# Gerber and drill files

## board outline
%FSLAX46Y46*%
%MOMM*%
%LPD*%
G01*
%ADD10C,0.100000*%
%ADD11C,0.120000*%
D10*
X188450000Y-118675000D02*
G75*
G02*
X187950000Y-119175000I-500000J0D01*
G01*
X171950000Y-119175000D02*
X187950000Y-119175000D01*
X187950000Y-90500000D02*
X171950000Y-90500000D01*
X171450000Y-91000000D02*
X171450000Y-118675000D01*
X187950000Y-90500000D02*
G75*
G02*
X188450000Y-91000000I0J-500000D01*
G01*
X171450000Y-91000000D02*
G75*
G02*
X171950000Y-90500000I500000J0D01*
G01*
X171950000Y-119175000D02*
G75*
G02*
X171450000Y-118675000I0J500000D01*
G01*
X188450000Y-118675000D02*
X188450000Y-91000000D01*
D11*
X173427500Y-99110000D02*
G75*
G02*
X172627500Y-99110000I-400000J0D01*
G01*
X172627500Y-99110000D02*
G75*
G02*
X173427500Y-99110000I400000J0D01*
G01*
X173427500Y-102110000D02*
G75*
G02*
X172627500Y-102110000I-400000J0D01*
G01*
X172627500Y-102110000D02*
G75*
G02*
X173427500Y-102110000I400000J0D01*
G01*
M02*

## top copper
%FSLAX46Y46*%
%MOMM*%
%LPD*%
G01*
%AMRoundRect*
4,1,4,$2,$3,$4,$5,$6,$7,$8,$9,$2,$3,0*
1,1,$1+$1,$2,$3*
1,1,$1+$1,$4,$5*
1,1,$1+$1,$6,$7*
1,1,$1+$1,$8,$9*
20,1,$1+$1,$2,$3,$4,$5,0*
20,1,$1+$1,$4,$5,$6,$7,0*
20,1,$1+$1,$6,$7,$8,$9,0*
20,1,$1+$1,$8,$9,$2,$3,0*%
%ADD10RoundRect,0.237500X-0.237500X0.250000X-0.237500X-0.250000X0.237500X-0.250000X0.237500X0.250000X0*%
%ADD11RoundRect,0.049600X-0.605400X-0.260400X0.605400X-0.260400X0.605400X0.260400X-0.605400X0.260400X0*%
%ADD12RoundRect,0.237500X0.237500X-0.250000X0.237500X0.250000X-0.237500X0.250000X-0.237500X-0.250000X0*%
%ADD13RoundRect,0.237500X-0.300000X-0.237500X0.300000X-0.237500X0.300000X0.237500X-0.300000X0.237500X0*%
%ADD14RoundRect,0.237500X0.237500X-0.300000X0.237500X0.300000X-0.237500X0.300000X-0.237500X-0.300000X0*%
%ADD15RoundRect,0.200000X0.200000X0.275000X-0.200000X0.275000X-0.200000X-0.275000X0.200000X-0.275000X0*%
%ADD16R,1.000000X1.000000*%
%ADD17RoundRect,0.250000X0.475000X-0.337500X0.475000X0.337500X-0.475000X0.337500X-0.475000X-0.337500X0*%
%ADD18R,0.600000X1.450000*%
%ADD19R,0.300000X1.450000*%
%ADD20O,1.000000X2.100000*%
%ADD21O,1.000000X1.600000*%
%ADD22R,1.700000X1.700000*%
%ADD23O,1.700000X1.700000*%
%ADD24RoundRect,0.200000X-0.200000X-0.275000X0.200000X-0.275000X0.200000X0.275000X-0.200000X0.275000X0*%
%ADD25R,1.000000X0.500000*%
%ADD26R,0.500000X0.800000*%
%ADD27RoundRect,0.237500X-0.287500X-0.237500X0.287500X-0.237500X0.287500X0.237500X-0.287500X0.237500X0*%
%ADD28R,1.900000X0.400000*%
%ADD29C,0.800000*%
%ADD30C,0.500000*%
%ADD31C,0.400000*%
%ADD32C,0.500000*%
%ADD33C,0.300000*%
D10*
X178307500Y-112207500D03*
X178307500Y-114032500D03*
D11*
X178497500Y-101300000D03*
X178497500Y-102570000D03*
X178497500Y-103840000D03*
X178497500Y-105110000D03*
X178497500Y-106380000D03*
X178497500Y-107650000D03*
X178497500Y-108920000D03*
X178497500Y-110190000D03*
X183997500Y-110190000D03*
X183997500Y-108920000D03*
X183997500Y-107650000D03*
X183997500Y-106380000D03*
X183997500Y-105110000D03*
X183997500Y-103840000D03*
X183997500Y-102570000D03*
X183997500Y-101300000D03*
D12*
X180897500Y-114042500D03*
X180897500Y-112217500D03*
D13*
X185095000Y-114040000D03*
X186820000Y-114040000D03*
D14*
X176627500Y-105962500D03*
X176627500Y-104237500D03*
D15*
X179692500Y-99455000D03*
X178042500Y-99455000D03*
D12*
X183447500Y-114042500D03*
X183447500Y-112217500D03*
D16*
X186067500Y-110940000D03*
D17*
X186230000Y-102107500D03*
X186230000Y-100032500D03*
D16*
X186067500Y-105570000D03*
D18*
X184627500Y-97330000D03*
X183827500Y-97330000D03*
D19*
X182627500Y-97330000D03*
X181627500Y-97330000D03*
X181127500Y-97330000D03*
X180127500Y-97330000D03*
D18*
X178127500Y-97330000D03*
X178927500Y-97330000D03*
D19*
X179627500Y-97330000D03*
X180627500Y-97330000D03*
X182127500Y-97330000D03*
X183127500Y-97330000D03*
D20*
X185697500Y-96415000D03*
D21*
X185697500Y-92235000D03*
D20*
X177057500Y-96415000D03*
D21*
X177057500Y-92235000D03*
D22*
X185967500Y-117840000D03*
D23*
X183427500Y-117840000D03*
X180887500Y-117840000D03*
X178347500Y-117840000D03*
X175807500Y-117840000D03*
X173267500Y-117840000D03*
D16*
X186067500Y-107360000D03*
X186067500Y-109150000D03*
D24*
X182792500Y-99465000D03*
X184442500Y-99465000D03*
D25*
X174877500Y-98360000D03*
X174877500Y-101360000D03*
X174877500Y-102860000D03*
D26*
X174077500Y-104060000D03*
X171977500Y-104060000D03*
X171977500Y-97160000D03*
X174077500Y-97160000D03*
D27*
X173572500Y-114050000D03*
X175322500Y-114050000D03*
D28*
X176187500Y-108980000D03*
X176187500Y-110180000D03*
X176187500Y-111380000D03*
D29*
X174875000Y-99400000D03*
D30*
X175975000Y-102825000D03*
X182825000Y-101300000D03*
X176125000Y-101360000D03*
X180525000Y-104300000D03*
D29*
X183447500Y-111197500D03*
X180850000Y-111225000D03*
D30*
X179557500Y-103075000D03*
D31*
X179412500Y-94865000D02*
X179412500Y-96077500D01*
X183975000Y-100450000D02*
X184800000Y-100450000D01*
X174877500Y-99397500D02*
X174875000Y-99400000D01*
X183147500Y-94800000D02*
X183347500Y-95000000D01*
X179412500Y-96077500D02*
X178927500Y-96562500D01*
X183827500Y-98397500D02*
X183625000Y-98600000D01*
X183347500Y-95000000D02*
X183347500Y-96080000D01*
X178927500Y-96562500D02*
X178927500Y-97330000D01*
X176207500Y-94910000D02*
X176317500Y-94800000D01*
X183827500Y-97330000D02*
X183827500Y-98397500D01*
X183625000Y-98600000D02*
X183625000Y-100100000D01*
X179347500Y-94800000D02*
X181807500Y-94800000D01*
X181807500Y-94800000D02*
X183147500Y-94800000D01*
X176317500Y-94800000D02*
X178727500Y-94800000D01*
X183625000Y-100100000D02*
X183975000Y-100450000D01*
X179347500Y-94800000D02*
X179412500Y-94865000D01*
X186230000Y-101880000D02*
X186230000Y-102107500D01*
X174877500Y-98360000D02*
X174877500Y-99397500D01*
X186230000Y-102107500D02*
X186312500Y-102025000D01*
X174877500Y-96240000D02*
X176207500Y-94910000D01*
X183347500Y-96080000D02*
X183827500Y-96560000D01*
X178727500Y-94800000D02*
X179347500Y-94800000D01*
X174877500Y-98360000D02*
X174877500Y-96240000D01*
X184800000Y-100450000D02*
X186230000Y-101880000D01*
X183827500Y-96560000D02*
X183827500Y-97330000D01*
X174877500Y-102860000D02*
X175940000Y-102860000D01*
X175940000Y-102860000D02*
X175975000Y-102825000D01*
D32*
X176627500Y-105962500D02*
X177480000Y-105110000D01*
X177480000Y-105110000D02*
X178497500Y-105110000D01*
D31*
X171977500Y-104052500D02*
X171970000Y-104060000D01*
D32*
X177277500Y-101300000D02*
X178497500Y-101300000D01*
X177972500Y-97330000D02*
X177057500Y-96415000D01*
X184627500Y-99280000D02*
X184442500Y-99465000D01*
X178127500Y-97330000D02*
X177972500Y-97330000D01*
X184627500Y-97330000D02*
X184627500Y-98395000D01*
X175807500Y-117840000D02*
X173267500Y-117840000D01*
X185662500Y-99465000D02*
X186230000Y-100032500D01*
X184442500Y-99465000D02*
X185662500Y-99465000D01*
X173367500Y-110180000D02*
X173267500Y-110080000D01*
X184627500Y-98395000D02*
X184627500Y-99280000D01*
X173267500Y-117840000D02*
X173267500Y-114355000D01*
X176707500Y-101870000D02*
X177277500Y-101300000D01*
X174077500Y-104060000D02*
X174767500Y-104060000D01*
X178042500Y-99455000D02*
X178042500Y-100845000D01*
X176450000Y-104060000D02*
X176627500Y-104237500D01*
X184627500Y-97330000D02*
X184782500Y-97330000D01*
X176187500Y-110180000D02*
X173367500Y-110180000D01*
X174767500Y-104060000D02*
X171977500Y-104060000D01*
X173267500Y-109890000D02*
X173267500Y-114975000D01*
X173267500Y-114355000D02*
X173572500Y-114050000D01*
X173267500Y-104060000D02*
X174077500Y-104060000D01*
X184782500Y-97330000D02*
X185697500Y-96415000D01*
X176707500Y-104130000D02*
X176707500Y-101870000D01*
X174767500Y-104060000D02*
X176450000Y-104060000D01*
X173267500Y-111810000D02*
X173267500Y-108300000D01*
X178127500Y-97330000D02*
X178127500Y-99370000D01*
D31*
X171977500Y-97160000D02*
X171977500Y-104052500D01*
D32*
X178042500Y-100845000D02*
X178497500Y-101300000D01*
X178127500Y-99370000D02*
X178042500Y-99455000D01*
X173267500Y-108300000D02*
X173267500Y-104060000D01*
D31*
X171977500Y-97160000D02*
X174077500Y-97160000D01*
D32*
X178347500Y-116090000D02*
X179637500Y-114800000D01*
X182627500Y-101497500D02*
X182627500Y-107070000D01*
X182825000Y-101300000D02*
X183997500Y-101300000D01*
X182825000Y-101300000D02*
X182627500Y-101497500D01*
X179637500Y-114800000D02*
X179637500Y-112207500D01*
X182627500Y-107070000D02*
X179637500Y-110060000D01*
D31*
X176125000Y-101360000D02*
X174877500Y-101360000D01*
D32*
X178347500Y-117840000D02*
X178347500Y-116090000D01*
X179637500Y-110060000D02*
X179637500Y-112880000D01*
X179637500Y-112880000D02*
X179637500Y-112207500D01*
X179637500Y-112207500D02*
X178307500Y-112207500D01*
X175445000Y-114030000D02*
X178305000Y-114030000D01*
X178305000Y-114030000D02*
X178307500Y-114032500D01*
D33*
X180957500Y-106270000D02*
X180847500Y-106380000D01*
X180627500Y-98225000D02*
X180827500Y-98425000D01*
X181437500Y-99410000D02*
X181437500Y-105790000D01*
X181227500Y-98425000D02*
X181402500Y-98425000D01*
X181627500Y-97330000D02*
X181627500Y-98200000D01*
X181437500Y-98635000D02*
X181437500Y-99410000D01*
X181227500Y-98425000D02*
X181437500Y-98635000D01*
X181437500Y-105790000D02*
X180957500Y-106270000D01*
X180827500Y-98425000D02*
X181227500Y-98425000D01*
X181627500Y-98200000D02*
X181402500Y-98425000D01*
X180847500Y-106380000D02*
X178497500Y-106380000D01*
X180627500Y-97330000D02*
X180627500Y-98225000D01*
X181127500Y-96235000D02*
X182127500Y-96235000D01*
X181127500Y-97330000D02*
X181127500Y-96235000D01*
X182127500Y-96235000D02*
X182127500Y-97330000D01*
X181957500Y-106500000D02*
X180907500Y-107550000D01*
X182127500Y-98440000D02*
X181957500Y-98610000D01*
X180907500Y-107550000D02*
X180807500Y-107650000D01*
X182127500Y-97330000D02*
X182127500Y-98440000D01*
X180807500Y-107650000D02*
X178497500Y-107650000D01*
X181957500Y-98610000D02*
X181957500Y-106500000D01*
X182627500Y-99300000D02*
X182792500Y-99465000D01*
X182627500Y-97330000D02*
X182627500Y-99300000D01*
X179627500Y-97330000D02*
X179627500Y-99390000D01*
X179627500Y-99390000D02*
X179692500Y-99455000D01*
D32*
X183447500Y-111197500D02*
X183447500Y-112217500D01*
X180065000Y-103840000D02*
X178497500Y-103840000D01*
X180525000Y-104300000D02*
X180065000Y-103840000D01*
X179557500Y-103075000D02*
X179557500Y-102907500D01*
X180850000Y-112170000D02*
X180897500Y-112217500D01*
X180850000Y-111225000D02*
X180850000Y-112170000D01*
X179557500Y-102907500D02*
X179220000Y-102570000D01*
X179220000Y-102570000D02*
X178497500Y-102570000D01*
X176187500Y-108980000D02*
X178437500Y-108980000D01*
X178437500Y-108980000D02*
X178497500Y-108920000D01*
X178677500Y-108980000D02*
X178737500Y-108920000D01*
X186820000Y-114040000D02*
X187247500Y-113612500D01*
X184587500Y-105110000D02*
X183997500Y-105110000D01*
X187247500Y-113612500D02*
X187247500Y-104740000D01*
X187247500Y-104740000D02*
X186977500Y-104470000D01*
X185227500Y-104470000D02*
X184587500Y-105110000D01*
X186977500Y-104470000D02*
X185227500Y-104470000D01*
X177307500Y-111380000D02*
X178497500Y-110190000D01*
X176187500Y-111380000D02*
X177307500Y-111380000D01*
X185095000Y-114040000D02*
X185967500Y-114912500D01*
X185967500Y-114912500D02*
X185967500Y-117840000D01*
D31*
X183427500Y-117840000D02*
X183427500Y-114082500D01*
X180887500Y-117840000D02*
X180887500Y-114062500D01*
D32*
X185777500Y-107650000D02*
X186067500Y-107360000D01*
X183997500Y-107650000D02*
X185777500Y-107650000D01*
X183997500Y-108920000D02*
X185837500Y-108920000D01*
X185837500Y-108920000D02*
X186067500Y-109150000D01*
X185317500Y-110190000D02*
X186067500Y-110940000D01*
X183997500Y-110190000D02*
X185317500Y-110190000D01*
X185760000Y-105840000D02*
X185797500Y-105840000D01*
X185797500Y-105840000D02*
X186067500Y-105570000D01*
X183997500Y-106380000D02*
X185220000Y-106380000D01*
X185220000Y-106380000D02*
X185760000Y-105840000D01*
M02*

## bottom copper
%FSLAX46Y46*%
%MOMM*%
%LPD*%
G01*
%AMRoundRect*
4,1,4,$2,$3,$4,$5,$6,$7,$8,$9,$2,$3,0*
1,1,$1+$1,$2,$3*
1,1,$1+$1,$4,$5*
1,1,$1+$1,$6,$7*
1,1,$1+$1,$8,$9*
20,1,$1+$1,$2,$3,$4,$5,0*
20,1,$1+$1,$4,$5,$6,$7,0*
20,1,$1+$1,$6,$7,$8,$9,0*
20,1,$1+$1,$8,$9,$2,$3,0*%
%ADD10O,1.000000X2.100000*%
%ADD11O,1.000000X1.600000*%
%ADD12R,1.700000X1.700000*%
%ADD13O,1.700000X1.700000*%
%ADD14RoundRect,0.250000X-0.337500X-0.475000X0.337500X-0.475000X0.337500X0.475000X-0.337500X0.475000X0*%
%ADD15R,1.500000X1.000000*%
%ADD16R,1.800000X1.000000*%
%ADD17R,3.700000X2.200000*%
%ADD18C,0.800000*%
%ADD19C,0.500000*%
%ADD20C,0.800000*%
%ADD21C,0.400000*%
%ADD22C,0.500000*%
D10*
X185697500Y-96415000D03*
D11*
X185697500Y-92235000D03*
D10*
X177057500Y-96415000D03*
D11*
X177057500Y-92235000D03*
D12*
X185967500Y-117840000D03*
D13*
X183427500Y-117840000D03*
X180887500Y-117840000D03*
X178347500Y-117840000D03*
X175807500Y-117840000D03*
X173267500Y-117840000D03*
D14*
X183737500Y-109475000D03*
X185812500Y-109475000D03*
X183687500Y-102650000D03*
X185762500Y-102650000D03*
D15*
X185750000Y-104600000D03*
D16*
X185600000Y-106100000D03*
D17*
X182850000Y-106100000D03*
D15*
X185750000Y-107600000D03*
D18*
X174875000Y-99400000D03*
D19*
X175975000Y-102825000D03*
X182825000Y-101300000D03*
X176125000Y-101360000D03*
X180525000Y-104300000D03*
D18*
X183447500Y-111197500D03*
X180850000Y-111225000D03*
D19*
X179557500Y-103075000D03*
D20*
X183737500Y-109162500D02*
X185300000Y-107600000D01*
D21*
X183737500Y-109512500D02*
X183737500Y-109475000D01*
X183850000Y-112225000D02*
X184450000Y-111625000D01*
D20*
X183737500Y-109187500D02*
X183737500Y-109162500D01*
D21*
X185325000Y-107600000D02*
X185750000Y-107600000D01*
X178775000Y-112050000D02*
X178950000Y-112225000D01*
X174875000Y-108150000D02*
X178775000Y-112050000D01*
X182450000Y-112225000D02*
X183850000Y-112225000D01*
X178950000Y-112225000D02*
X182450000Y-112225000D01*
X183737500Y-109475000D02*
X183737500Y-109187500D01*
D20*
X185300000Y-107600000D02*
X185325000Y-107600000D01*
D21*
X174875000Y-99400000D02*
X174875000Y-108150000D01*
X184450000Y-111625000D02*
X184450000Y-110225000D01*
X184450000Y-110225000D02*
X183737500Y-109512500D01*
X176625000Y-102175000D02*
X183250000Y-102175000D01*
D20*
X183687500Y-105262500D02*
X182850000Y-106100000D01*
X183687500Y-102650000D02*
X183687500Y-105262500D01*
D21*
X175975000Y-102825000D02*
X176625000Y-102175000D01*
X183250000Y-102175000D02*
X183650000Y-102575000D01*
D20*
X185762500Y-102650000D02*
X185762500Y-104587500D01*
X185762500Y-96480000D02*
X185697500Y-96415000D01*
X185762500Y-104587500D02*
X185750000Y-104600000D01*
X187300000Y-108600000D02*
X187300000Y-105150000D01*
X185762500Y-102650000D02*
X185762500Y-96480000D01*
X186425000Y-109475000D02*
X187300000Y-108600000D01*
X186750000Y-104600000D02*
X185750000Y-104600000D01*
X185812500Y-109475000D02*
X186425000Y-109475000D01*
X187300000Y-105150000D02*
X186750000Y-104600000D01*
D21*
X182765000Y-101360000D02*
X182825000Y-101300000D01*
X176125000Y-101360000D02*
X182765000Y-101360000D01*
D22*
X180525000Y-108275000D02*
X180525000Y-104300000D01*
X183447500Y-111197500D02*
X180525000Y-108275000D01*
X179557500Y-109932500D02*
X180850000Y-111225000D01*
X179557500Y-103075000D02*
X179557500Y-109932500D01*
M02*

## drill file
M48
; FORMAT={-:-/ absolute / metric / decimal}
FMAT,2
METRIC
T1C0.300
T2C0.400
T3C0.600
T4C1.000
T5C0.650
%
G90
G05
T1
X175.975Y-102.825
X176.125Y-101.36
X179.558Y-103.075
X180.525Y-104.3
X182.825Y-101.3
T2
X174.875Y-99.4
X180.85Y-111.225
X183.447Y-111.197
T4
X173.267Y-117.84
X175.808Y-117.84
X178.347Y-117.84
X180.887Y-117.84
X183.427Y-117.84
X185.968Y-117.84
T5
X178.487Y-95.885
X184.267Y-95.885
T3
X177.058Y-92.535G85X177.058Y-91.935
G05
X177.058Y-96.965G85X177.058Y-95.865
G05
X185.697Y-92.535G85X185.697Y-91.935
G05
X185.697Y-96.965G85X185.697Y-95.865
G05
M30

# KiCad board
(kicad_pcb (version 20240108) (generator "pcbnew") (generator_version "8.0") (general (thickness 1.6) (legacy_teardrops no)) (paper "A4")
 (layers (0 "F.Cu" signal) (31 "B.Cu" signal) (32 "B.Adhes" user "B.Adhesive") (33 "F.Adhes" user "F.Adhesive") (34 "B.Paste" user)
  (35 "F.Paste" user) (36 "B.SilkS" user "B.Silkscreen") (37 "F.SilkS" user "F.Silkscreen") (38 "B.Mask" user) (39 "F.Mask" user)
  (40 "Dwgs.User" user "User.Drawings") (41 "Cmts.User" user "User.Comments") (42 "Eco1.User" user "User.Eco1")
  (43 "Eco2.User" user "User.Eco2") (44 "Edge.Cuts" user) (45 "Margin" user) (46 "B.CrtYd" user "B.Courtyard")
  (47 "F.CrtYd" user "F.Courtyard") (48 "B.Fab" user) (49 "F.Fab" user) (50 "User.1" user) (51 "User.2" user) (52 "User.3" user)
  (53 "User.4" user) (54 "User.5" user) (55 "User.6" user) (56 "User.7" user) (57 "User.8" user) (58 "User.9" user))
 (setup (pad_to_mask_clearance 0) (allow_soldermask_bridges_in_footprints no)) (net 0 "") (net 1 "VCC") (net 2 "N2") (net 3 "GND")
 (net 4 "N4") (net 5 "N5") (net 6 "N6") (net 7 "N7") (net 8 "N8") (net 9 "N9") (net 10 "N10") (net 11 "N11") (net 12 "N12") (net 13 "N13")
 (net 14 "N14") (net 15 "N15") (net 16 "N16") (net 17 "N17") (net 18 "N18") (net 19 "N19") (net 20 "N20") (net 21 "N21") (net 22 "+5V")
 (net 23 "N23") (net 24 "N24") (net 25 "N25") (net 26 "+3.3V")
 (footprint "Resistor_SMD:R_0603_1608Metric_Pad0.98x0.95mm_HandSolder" (layer "F.Cu") (at 178.3075 113.12 -90)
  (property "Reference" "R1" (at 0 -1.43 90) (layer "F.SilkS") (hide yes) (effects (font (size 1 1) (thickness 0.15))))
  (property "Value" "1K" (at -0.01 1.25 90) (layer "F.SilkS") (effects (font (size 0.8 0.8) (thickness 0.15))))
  (pad "1" smd roundrect (at -0.9125 0 270) (size 0.975 0.95) (layers "F.Cu" "F.Paste" "F.Mask") (roundrect_rratio 0.25) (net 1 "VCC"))
  (pad "2" smd roundrect (at 0.9125 0 270) (size 0.975 0.95) (layers "F.Cu" "F.Paste" "F.Mask") (roundrect_rratio 0.25) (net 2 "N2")))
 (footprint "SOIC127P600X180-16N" (layer "F.Cu") (at 181.2475 105.745)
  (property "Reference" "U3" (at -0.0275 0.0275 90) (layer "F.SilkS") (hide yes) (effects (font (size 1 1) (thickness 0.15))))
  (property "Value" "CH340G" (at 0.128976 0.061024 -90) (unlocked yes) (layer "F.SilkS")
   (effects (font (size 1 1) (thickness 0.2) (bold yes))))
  (pad "1" smd roundrect (at -2.75 -4.445) (size 1.31 0.62) (layers "F.Cu" "F.Paste" "F.Mask") (roundrect_rratio 0.08) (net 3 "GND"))
  (pad "2" smd roundrect (at -2.75 -3.175) (size 1.31 0.62) (layers "F.Cu" "F.Paste" "F.Mask") (roundrect_rratio 0.08) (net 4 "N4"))
  (pad "3" smd roundrect (at -2.75 -1.905) (size 1.31 0.62) (layers "F.Cu" "F.Paste" "F.Mask") (roundrect_rratio 0.08) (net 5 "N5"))
  (pad "4" smd roundrect (at -2.75 -0.635) (size 1.31 0.62) (layers "F.Cu" "F.Paste" "F.Mask") (roundrect_rratio 0.08) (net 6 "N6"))
  (pad "5" smd roundrect (at -2.75 0.635) (size 1.31 0.62) (layers "F.Cu" "F.Paste" "F.Mask") (roundrect_rratio 0.08) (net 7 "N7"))
  (pad "6" smd roundrect (at -2.75 1.905) (size 1.31 0.62) (layers "F.Cu" "F.Paste" "F.Mask") (roundrect_rratio 0.08) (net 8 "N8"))
  (pad "7" smd roundrect (at -2.75 3.175) (size 1.31 0.62) (layers "F.Cu" "F.Paste" "F.Mask") (roundrect_rratio 0.08) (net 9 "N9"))
  (pad "8" smd roundrect (at -2.75 4.445) (size 1.31 0.62) (layers "F.Cu" "F.Paste" "F.Mask") (roundrect_rratio 0.08) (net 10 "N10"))
  (pad "9" smd roundrect (at 2.75 4.445) (size 1.31 0.62) (layers "F.Cu" "F.Paste" "F.Mask") (roundrect_rratio 0.08) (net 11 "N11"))
  (pad "10" smd roundrect (at 2.75 3.175) (size 1.31 0.62) (layers "F.Cu" "F.Paste" "F.Mask") (roundrect_rratio 0.08) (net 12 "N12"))
  (pad "11" smd roundrect (at 2.75 1.905) (size 1.31 0.62) (layers "F.Cu" "F.Paste" "F.Mask") (roundrect_rratio 0.08) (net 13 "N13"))
  (pad "12" smd roundrect (at 2.75 0.635) (size 1.31 0.62) (layers "F.Cu" "F.Paste" "F.Mask") (roundrect_rratio 0.08) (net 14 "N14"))
  (pad "13" smd roundrect (at 2.75 -0.635) (size 1.31 0.62) (layers "F.Cu" "F.Paste" "F.Mask") (roundrect_rratio 0.08) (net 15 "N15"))
  (pad "14" smd roundrect (at 2.75 -1.905) (size 1.31 0.62) (layers "F.Cu" "F.Paste" "F.Mask") (roundrect_rratio 0.08) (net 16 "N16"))
  (pad "15" smd roundrect (at 2.75 -3.175) (size 1.31 0.62) (layers "F.Cu" "F.Paste" "F.Mask") (roundrect_rratio 0.08) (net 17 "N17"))
  (pad "16" smd roundrect (at 2.75 -4.445) (size 1.31 0.62) (layers "F.Cu" "F.Paste" "F.Mask") (roundrect_rratio 0.08) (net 1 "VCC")))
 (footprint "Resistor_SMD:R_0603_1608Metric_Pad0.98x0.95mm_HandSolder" (layer "F.Cu") (at 180.8975 113.13 90)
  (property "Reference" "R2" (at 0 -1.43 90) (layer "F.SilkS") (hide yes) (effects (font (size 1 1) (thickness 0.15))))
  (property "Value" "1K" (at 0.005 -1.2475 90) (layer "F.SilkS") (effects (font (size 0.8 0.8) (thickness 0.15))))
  (pad "1" smd roundrect (at -0.9125 0 90) (size 0.975 0.95) (layers "F.Cu" "F.Paste" "F.Mask") (roundrect_rratio 0.25) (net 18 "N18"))
  (pad "2" smd roundrect (at 0.9125 0 90) (size 0.975 0.95) (layers "F.Cu" "F.Paste" "F.Mask") (roundrect_rratio 0.25) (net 4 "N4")))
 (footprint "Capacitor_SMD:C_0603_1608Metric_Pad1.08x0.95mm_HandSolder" (layer "F.Cu") (at 185.9575 114.04)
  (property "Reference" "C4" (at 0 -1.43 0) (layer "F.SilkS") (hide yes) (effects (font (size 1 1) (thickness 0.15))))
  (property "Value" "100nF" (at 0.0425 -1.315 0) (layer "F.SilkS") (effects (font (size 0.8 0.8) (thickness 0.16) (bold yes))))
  (pad "1" smd roundrect (at -0.8625 0) (size 1.075 0.95) (layers "F.Cu" "F.Paste" "F.Mask") (roundrect_rratio 0.25) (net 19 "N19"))
  (pad "2" smd roundrect (at 0.8625 0) (size 1.075 0.95) (layers "F.Cu" "F.Paste" "F.Mask") (roundrect_rratio 0.25) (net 15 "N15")))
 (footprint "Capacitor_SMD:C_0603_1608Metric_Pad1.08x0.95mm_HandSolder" (layer "F.Cu") (at 176.6275 105.1 90)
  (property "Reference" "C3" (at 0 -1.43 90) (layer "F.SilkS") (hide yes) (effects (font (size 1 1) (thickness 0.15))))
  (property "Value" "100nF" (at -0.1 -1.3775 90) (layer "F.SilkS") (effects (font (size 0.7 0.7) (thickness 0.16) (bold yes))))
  (pad "1" smd roundrect (at -0.8625 0 90) (size 1.075 0.95) (layers "F.Cu" "F.Paste" "F.Mask") (roundrect_rratio 0.25) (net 6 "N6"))
  (pad "2" smd roundrect (at 0.8625 0 90) (size 1.075 0.95) (layers "F.Cu" "F.Paste" "F.Mask") (roundrect_rratio 0.25) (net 3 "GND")))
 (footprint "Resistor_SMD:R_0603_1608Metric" (layer "F.Cu") (at 178.8675 99.455 180)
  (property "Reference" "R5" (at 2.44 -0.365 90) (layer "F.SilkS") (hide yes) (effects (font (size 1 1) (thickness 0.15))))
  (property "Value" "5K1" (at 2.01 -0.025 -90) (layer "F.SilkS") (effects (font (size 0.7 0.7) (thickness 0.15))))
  (pad "1" smd roundrect (at -0.825 0 180) (size 0.8 0.95) (layers "F.Cu" "F.Paste" "F.Mask") (roundrect_rratio 0.25) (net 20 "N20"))
  (pad "2" smd roundrect (at 0.825 0 180) (size 0.8 0.95) (layers "F.Cu" "F.Paste" "F.Mask") (roundrect_rratio 0.25) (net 3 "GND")))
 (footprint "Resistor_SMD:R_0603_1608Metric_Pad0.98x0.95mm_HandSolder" (layer "F.Cu") (at 183.4475 113.13 90)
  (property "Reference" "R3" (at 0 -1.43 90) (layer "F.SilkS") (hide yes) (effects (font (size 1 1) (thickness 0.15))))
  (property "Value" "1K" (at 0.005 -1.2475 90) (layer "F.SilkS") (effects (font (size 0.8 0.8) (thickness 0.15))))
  (pad "1" smd roundrect (at -0.9125 0 90) (size 0.975 0.95) (layers "F.Cu" "F.Paste" "F.Mask") (roundrect_rratio 0.25) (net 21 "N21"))
  (pad "2" smd roundrect (at 0.9125 0 90) (size 0.975 0.95) (layers "F.Cu" "F.Paste" "F.Mask") (roundrect_rratio 0.25) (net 5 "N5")))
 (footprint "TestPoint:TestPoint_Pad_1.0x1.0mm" (layer "F.Cu") (at 186.0675 110.94)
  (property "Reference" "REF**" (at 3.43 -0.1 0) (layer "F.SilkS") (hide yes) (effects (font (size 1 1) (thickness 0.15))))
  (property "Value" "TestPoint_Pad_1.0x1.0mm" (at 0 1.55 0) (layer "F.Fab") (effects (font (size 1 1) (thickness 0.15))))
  (pad "1" smd rect (at 0 0) (size 1 1) (layers "F.Cu" "F.Mask") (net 11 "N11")))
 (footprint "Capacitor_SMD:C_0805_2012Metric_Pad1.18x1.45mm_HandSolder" (layer "F.Cu") (at 186.23 101.07 90)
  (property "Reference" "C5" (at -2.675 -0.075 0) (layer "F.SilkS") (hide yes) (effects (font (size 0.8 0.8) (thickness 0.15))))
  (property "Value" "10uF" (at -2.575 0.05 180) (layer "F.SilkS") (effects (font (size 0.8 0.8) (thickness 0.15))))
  (pad "1" smd roundrect (at -1.0375 0 90) (size 1.175 1.45) (layers "F.Cu" "F.Paste" "F.Mask") (roundrect_rratio 0.212766) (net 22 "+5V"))
  (pad "2" smd roundrect (at 1.0375 0 90) (size 1.175 1.45) (layers "F.Cu" "F.Paste" "F.Mask") (roundrect_rratio 0.212766) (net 3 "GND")))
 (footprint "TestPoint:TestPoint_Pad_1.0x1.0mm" (layer "F.Cu") (at 186.0675 105.57)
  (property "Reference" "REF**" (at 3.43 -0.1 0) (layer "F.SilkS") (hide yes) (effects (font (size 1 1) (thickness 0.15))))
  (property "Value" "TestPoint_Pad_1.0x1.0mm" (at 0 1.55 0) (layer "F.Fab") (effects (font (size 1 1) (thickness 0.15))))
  (pad "1" smd rect (at 0 0) (size 1 1) (layers "F.Cu" "F.Mask") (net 14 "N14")))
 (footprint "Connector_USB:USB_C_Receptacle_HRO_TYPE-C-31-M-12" (layer "F.Cu") (at 181.3775 93.285 180)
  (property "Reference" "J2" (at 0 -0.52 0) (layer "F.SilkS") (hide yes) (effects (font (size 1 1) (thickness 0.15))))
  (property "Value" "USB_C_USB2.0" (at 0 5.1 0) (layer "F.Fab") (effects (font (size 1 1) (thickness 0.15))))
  (pad "" np_thru_hole circle (at -2.89 -2.6 180) (size 0.65 0.65) (drill 0.65) (layers "F&B.Cu" "*.Mask"))
  (pad "" np_thru_hole circle (at 2.89 -2.6 180) (size 0.65 0.65) (drill 0.65) (layers "F&B.Cu" "*.Mask"))
  (pad "A1" smd rect (at -3.25 -4.045 180) (size 0.6 1.45) (layers "F.Cu" "F.Paste" "F.Mask") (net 3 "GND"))
  (pad "A4" smd rect (at -2.45 -4.045 180) (size 0.6 1.45) (layers "F.Cu" "F.Paste" "F.Mask") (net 22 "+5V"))
  (pad "A5" smd rect (at -1.25 -4.045 180) (size 0.3 1.45) (layers "F.Cu" "F.Paste" "F.Mask") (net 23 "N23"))
  (pad "A6" smd rect (at -0.25 -4.045 180) (size 0.3 1.45) (layers "F.Cu" "F.Paste" "F.Mask") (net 7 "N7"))
  (pad "A7" smd rect (at 0.25 -4.045 180) (size 0.3 1.45) (layers "F.Cu" "F.Paste" "F.Mask") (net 8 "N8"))
  (pad "A8" smd rect (at 1.25 -4.045 180) (size 0.3 1.45) (layers "F.Cu" "F.Paste" "F.Mask") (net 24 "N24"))
  (pad "B1" smd rect (at 3.25 -4.045 180) (size 0.6 1.45) (layers "F.Cu" "F.Paste" "F.Mask") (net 3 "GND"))
  (pad "B4" smd rect (at 2.45 -4.045 180) (size 0.6 1.45) (layers "F.Cu" "F.Paste" "F.Mask") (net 22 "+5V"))
  (pad "B5" smd rect (at 1.75 -4.045 180) (size 0.3 1.45) (layers "F.Cu" "F.Paste" "F.Mask") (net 20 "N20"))
  (pad "B6" smd rect (at 0.75 -4.045 180) (size 0.3 1.45) (layers "F.Cu" "F.Paste" "F.Mask") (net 7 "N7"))
  (pad "B7" smd rect (at -0.75 -4.045 180) (size 0.3 1.45) (layers "F.Cu" "F.Paste" "F.Mask") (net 8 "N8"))
  (pad "B8" smd rect (at -1.75 -4.045 180) (size 0.3 1.45) (layers "F.Cu" "F.Paste" "F.Mask") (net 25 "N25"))
  (pad "S1" thru_hole oval (at -4.32 -3.13 180) (size 1 2.1) (drill oval 0.6 1.7) (layers "*.Cu" "*.Mask") (remove_unused_layers no)
   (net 3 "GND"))
  (pad "S1" thru_hole oval (at -4.32 1.05 180) (size 1 1.6) (drill oval 0.6 1.2) (layers "*.Cu" "*.Mask") (remove_unused_layers no)
   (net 3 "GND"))
  (pad "S1" thru_hole oval (at 4.32 -3.13 180) (size 1 2.1) (drill oval 0.6 1.7) (layers "*.Cu" "*.Mask") (remove_unused_layers no)
   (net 3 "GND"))
  (pad "S1" thru_hole oval (at 4.32 1.05 180) (size 1 1.6) (drill oval 0.6 1.2) (layers "*.Cu" "*.Mask") (remove_unused_layers no)
   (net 3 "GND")))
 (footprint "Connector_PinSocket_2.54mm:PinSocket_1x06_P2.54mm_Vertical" (layer "F.Cu") (at 185.9675 117.84 -90)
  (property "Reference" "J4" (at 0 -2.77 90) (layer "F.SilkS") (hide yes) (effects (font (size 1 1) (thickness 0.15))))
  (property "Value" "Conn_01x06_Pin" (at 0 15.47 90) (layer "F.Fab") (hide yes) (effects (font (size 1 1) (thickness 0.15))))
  (pad "1" thru_hole rect (at 0 0 270) (size 1.7 1.7) (drill 1) (layers "*.Cu" "*.Mask") (remove_unused_layers no) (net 19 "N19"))
  (pad "2" thru_hole oval (at 0 2.54 270) (size 1.7 1.7) (drill 1) (layers "*.Cu" "*.Mask") (remove_unused_layers no) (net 21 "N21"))
  (pad "3" thru_hole oval (at 0 5.08 270) (size 1.7 1.7) (drill 1) (layers "*.Cu" "*.Mask") (remove_unused_layers no) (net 18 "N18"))
  (pad "4" thru_hole oval (at 0 7.62 270) (size 1.7 1.7) (drill 1) (layers "*.Cu" "*.Mask") (remove_unused_layers no) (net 1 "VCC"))
  (pad "5" thru_hole oval (at 0 10.16 270) (size 1.7 1.7) (drill 1) (layers "*.Cu" "*.Mask") (remove_unused_layers no) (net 3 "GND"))
  (pad "6" thru_hole oval (at 0 12.7 270) (size 1.7 1.7) (drill 1) (layers "*.Cu" "*.Mask") (remove_unused_layers no) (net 3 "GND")))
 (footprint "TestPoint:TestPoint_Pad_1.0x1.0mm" (layer "F.Cu") (at 186.0675 107.36)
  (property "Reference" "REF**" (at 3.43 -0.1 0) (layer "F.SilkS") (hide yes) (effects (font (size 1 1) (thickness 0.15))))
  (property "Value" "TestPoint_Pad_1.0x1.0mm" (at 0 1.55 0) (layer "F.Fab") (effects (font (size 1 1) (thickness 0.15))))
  (pad "1" smd rect (at 0 0) (size 1 1) (layers "F.Cu" "F.Mask") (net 13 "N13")))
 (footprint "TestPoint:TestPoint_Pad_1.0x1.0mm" (layer "F.Cu") (at 186.0675 109.15)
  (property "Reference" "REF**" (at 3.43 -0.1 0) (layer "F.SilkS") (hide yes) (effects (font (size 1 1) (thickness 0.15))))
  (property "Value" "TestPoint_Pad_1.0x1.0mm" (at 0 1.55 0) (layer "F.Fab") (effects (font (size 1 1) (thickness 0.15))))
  (pad "1" smd rect (at 0 0) (size 1 1) (layers "F.Cu" "F.Mask") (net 12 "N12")))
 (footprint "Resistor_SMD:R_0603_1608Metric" (layer "F.Cu") (at 183.6175 99.465)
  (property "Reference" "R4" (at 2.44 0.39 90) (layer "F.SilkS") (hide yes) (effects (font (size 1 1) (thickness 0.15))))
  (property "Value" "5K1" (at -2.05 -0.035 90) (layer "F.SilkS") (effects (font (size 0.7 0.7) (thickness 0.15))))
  (pad "1" smd roundrect (at -0.825 0) (size 0.8 0.95) (layers "F.Cu" "F.Paste" "F.Mask") (roundrect_rratio 0.25) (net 23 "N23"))
  (pad "2" smd roundrect (at 0.825 0) (size 0.8 0.95) (layers "F.Cu" "F.Paste" "F.Mask") (roundrect_rratio 0.25) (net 3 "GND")))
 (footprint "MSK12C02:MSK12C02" (layer "F.Cu") (at 173.0275 100.61 -90)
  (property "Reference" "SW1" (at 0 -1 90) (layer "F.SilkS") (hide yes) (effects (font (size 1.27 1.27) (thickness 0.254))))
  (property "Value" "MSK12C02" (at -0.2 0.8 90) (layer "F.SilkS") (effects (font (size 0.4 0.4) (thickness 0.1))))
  (fp_circle (center -1.5 0) (end -1.1 0) (stroke (width 0.12) (type solid)) (fill none) (layer "Edge.Cuts"))
  (fp_circle (center 1.5 0) (end 1.9 0) (stroke (width 0.12) (type solid)) (fill none) (layer "Edge.Cuts"))
  (pad "A1" smd rect (at -2.25 -1.85 270) (size 0.5 1) (layers "F.Cu" "F.Paste" "F.Mask") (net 22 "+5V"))
  (pad "B1" smd rect (at 0.75 -1.85 270) (size 0.5 1) (layers "F.Cu" "F.Paste" "F.Mask") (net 1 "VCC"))
  (pad "C1" smd rect (at 2.25 -1.85 270) (size 0.5 1) (layers "F.Cu" "F.Paste" "F.Mask") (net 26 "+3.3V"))
  (pad "MP1" smd rect (at 3.45 -1.05) (size 0.5 0.8) (layers "F.Cu" "F.Paste" "F.Mask") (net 3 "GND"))
  (pad "MP2" smd rect (at 3.45 1.05) (size 0.5 0.8) (layers "F.Cu" "F.Paste" "F.Mask") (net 3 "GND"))
  (pad "MP3" smd rect (at -3.45 1.05) (size 0.5 0.8) (layers "F.Cu" "F.Paste" "F.Mask") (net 3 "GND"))
  (pad "MP4" smd rect (at -3.45 -1.05) (size 0.5 0.8) (layers "F.Cu" "F.Paste" "F.Mask") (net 3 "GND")))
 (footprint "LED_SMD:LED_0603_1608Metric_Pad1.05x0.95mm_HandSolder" (layer "F.Cu") (at 174.4475 114.05)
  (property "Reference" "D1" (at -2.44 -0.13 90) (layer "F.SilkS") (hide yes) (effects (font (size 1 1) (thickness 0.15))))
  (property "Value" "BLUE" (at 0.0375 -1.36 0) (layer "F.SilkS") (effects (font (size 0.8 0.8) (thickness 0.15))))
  (pad "1" smd roundrect (at -0.875 0) (size 1.05 0.95) (layers "F.Cu" "F.Paste" "F.Mask") (roundrect_rratio 0.25) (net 3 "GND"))
  (pad "2" smd roundrect (at 0.875 0) (size 1.05 0.95) (layers "F.Cu" "F.Paste" "F.Mask") (roundrect_rratio 0.25) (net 2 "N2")))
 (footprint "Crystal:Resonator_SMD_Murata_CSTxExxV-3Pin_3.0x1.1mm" (layer "F.Cu") (at 176.1875 110.18 -90)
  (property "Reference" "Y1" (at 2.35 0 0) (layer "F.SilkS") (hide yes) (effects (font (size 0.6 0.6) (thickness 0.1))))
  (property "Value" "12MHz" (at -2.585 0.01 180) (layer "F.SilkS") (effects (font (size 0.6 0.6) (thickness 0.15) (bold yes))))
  (pad "1" smd rect (at -1.2 0 270) (size 0.4 1.9) (layers "F.Cu" "F.Paste" "F.Mask") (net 9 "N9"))
  (pad "2" smd rect (at 0 0 270) (size 0.4 1.9) (layers "F.Cu" "F.Paste" "F.Mask") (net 3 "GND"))
  (pad "3" smd rect (at 1.2 0 270) (size 0.4 1.9) (layers "F.Cu" "F.Paste" "F.Mask") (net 10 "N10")))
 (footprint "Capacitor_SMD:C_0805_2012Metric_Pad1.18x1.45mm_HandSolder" (layer "B.Cu") (at 184.775 109.475)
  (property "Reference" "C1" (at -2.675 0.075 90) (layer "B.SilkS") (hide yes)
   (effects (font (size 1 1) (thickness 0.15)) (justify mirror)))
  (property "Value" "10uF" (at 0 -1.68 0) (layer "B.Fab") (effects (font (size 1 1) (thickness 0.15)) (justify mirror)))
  (pad "1" smd roundrect (at -1.0375 0) (size 1.175 1.45) (layers "B.Cu" "B.Paste" "B.Mask") (roundrect_rratio 0.212766) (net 22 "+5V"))
  (pad "2" smd roundrect (at 1.0375 0) (size 1.175 1.45) (layers "B.Cu" "B.Paste" "B.Mask") (roundrect_rratio 0.212766) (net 3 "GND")))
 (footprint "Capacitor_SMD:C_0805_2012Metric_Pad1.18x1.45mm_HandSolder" (layer "B.Cu") (at 184.725 102.65)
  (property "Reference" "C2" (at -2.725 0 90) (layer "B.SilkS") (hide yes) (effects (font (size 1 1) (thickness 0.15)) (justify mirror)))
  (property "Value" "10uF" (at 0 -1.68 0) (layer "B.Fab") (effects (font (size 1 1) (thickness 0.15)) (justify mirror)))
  (pad "1" smd roundrect (at -1.0375 0) (size 1.175 1.45) (layers "B.Cu" "B.Paste" "B.Mask") (roundrect_rratio 0.212766) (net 26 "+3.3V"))
  (pad "2" smd roundrect (at 1.0375 0) (size 1.175 1.45) (layers "B.Cu" "B.Paste" "B.Mask") (roundrect_rratio 0.212766) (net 3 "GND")))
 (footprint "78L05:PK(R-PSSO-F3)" (layer "B.Cu") (at 182.1 106.1 -90)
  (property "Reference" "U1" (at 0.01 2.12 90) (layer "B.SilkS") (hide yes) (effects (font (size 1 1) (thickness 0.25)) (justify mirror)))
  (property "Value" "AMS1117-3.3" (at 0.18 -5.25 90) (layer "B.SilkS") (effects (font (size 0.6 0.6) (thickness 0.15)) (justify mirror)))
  (pad "1" smd rect (at -1.5 -3.65 270) (size 1 1.5) (layers "B.Cu" "B.Paste" "B.Mask") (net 3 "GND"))
  (pad "2" smd rect (at 0 -3.5 270) (size 1 1.8) (layers "B.Cu" "B.Paste" "B.Mask") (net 26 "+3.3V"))
  (pad "2" smd rect (at 0 -0.75 270) (size 2.2 3.7) (layers "B.Cu" "B.Paste" "B.Mask") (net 26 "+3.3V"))
  (pad "3" smd rect (at 1.5 -3.65 270) (size 1 1.5) (layers "B.Cu" "B.Paste" "B.Mask") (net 22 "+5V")))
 (gr_arc (start 188.45 118.675) (mid 188.303553 119.028553) (end 187.95 119.175) (stroke (width 0.1) (type solid)) (layer "Edge.Cuts"))
 (gr_line (start 171.95 119.175) (end 187.95 119.175) (stroke (width 0.1) (type default)) (layer "Edge.Cuts"))
 (gr_line (start 187.95 90.5) (end 171.95 90.5) (stroke (width 0.1) (type default)) (layer "Edge.Cuts"))
 (gr_line (start 171.45 91) (end 171.45 118.675) (stroke (width 0.1) (type default)) (layer "Edge.Cuts"))
 (gr_arc (start 187.95 90.5) (mid 188.303553 90.646447) (end 188.45 91) (stroke (width 0.1) (type solid)) (layer "Edge.Cuts"))
 (gr_arc (start 171.45 91) (mid 171.596447 90.646447) (end 171.95 90.5) (stroke (width 0.1) (type solid)) (layer "Edge.Cuts"))
 (gr_arc (start 171.95 119.175) (mid 171.596447 119.028553) (end 171.45 118.675) (stroke (width 0.1) (type solid)) (layer "Edge.Cuts"))
 (gr_line (start 188.45 118.675) (end 188.45 91) (stroke (width 0.1) (type default)) (layer "Edge.Cuts"))
 (segment (start 179.4125 94.865) (end 179.4125 96.0775) (width 0.4) (layer "F.Cu") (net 22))
 (segment (start 183.975 100.45) (end 184.8 100.45) (width 0.4) (layer "F.Cu") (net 22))
 (segment (start 174.8775 99.3975) (end 174.875 99.4) (width 0.4) (layer "F.Cu") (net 22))
 (segment (start 183.1475 94.8) (end 183.3475 95) (width 0.4) (layer "F.Cu") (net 22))
 (segment (start 179.4125 96.0775) (end 178.9275 96.5625) (width 0.4) (layer "F.Cu") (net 22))
 (segment (start 183.8275 98.3975) (end 183.625 98.6) (width 0.4) (layer "F.Cu") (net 22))
 (segment (start 183.3475 95) (end 183.3475 96.08) (width 0.4) (layer "F.Cu") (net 22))
 (segment (start 178.9275 96.5625) (end 178.9275 97.33) (width 0.4) (layer "F.Cu") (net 22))
 (segment (start 176.2075 94.91) (end 176.3175 94.8) (width 0.4) (layer "F.Cu") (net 22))
 (segment (start 183.8275 97.33) (end 183.8275 98.3975) (width 0.4) (layer "F.Cu") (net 22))
 (segment (start 183.625 98.6) (end 183.625 100.1) (width 0.4) (layer "F.Cu") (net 22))
 (segment (start 179.3475 94.8) (end 181.8075 94.8) (width 0.4) (layer "F.Cu") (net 22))
 (segment (start 181.8075 94.8) (end 183.1475 94.8) (width 0.4) (layer "F.Cu") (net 22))
 (segment (start 176.3175 94.8) (end 178.7275 94.8) (width 0.4) (layer "F.Cu") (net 22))
 (segment (start 183.625 100.1) (end 183.975 100.45) (width 0.4) (layer "F.Cu") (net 22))
 (segment (start 179.3475 94.8) (end 179.4125 94.865) (width 0.4) (layer "F.Cu") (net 22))
 (segment (start 186.23 101.88) (end 186.23 102.1075) (width 0.4) (layer "F.Cu") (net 22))
 (segment (start 174.8775 98.36) (end 174.8775 99.3975) (width 0.4) (layer "F.Cu") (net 22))
 (segment (start 186.23 102.1075) (end 186.3125 102.025) (width 0.4) (layer "F.Cu") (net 22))
 (segment (start 174.8775 96.24) (end 176.2075 94.91) (width 0.4) (layer "F.Cu") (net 22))
 (segment (start 183.3475 96.08) (end 183.8275 96.56) (width 0.4) (layer "F.Cu") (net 22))
 (segment (start 178.7275 94.8) (end 179.3475 94.8) (width 0.4) (layer "F.Cu") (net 22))
 (segment (start 174.8775 98.36) (end 174.8775 96.24) (width 0.4) (layer "F.Cu") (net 22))
 (segment (start 184.8 100.45) (end 186.23 101.88) (width 0.4) (layer "F.Cu") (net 22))
 (segment (start 183.8275 96.56) (end 183.8275 97.33) (width 0.4) (layer "F.Cu") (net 22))
 (via (at 174.875 99.4) (size 0.8) (drill 0.4) (layers "F.Cu" "B.Cu") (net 22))
 (segment (start 183.7375 109.1625) (end 185.3 107.6) (width 0.8) (layer "B.Cu") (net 22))
 (segment (start 183.7375 109.5125) (end 183.7375 109.475) (width 0.4) (layer "B.Cu") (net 22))
 (segment (start 183.85 112.225) (end 184.45 111.625) (width 0.4) (layer "B.Cu") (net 22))
 (segment (start 183.7375 109.1875) (end 183.7375 109.1625) (width 0.8) (layer "B.Cu") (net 22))
 (segment (start 185.325 107.6) (end 185.75 107.6) (width 0.4) (layer "B.Cu") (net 22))
 (segment (start 178.775 112.05) (end 178.95 112.225) (width 0.4) (layer "B.Cu") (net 22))
 (segment (start 174.875 108.15) (end 178.775 112.05) (width 0.4) (layer "B.Cu") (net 22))
 (segment (start 182.45 112.225) (end 183.85 112.225) (width 0.4) (layer "B.Cu") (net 22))
 (segment (start 178.95 112.225) (end 182.45 112.225) (width 0.4) (layer "B.Cu") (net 22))
 (segment (start 183.7375 109.475) (end 183.7375 109.1875) (width 0.4) (layer "B.Cu") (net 22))
 (segment (start 185.3 107.6) (end 185.325 107.6) (width 0.8) (layer "B.Cu") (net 22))
 (segment (start 174.875 99.4) (end 174.875 108.15) (width 0.4) (layer "B.Cu") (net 22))
 (segment (start 184.45 111.625) (end 184.45 110.225) (width 0.4) (layer "B.Cu") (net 22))
 (segment (start 184.45 110.225) (end 183.7375 109.5125) (width 0.4) (layer "B.Cu") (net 22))
 (segment (start 174.8775 102.86) (end 175.94 102.86) (width 0.4) (layer "F.Cu") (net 26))
 (segment (start 175.94 102.86) (end 175.975 102.825) (width 0.4) (layer "F.Cu") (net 26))
 (via (at 175.975 102.825) (size 0.5) (drill 0.3) (layers "F.Cu" "B.Cu") (free yes) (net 26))
 (segment (start 176.625 102.175) (end 183.25 102.175) (width 0.4) (layer "B.Cu") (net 26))
 (segment (start 183.6875 105.2625) (end 182.85 106.1) (width 0.8) (layer "B.Cu") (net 26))
 (segment (start 183.6875 102.65) (end 183.6875 105.2625) (width 0.8) (layer "B.Cu") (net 26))
 (segment (start 175.975 102.825) (end 176.625 102.175) (width 0.4) (layer "B.Cu") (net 26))
 (segment (start 183.25 102.175) (end 183.65 102.575) (width 0.4) (layer "B.Cu") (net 26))
 (segment (start 176.6275 105.9625) (end 177.48 105.11) (width 0.5) (layer "F.Cu") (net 6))
 (segment (start 177.48 105.11) (end 178.4975 105.11) (width 0.5) (layer "F.Cu") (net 6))
 (segment (start 171.9775 104.0525) (end 171.97 104.06) (width 0.4) (layer "F.Cu") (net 3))
 (segment (start 177.2775 101.3) (end 178.4975 101.3) (width 0.5) (layer "F.Cu") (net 3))
 (segment (start 177.9725 97.33) (end 177.0575 96.415) (width 0.5) (layer "F.Cu") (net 3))
 (segment (start 184.6275 99.28) (end 184.4425 99.465) (width 0.5) (layer "F.Cu") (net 3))
 (segment (start 178.1275 97.33) (end 177.9725 97.33) (width 0.5) (layer "F.Cu") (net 3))
 (segment (start 184.6275 97.33) (end 184.6275 98.395) (width 0.5) (layer "F.Cu") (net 3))
 (segment (start 175.8075 117.84) (end 173.2675 117.84) (width 0.5) (layer "F.Cu") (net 3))
 (segment (start 185.6625 99.465) (end 186.23 100.0325) (width 0.5) (layer "F.Cu") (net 3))
 (segment (start 184.4425 99.465) (end 185.6625 99.465) (width 0.5) (layer "F.Cu") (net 3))
 (segment (start 173.3675 110.18) (end 173.2675 110.08) (width 0.5) (layer "F.Cu") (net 3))
 (segment (start 184.6275 98.395) (end 184.6275 99.28) (width 0.5) (layer "F.Cu") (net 3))
 (segment (start 173.2675 117.84) (end 173.2675 114.355) (width 0.5) (layer "F.Cu") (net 3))
 (segment (start 176.7075 101.87) (end 177.2775 101.3) (width 0.5) (layer "F.Cu") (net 3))
 (segment (start 174.0775 104.06) (end 174.7675 104.06) (width 0.5) (layer "F.Cu") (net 3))
 (segment (start 178.0425 99.455) (end 178.0425 100.845) (width 0.5) (layer "F.Cu") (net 3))
 (segment (start 176.45 104.06) (end 176.6275 104.2375) (width 0.5) (layer "F.Cu") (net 3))
 (segment (start 184.6275 97.33) (end 184.7825 97.33) (width 0.5) (layer "F.Cu") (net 3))
 (segment (start 176.1875 110.18) (end 173.3675 110.18) (width 0.5) (layer "F.Cu") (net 3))
 (segment (start 174.7675 104.06) (end 171.9775 104.06) (width 0.5) (layer "F.Cu") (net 3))
 (segment (start 173.2675 109.89) (end 173.2675 114.975) (width 0.5) (layer "F.Cu") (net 3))
 (segment (start 173.2675 114.355) (end 173.5725 114.05) (width 0.5) (layer "F.Cu") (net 3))
 (segment (start 173.2675 104.06) (end 174.0775 104.06) (width 0.5) (layer "F.Cu") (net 3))
 (segment (start 184.7825 97.33) (end 185.6975 96.415) (width 0.5) (layer "F.Cu") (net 3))
 (segment (start 176.7075 104.13) (end 176.7075 101.87) (width 0.5) (layer "F.Cu") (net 3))
 (segment (start 174.7675 104.06) (end 176.45 104.06) (width 0.5) (layer "F.Cu") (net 3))
 (segment (start 173.2675 111.81) (end 173.2675 108.3) (width 0.5) (layer "F.Cu") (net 3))
 (segment (start 178.1275 97.33) (end 178.1275 99.37) (width 0.5) (layer "F.Cu") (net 3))
 (segment (start 171.9775 97.16) (end 171.9775 104.0525) (width 0.4) (layer "F.Cu") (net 3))
 (segment (start 178.0425 100.845) (end 178.4975 101.3) (width 0.5) (layer "F.Cu") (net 3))
 (segment (start 178.1275 99.37) (end 178.0425 99.455) (width 0.5) (layer "F.Cu") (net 3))
 (segment (start 173.2675 108.3) (end 173.2675 104.06) (width 0.5) (layer "F.Cu") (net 3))
 (segment (start 171.9775 97.16) (end 174.0775 97.16) (width 0.4) (layer "F.Cu") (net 3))
 (segment (start 185.7625 102.65) (end 185.7625 104.5875) (width 0.8) (layer "B.Cu") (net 3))
 (segment (start 185.7625 96.48) (end 185.6975 96.415) (width 0.8) (layer "B.Cu") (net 3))
 (segment (start 185.7625 104.5875) (end 185.75 104.6) (width 0.8) (layer "B.Cu") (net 3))
 (segment (start 187.3 108.6) (end 187.3 105.15) (width 0.8) (layer "B.Cu") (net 3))
 (segment (start 185.7625 102.65) (end 185.7625 96.48) (width 0.8) (layer "B.Cu") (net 3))
 (segment (start 186.425 109.475) (end 187.3 108.6) (width 0.8) (layer "B.Cu") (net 3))
 (segment (start 186.75 104.6) (end 185.75 104.6) (width 0.8) (layer "B.Cu") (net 3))
 (segment (start 185.8125 109.475) (end 186.425 109.475) (width 0.8) (layer "B.Cu") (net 3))
 (segment (start 187.3 105.15) (end 186.75 104.6) (width 0.8) (layer "B.Cu") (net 3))
 (segment (start 178.3475 116.09) (end 179.6375 114.8) (width 0.5) (layer "F.Cu") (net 1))
 (segment (start 182.6275 101.4975) (end 182.6275 107.07) (width 0.5) (layer "F.Cu") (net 1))
 (segment (start 182.825 101.3) (end 183.9975 101.3) (width 0.5) (layer "F.Cu") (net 1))
 (segment (start 182.825 101.3) (end 182.6275 101.4975) (width 0.5) (layer "F.Cu") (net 1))
 (segment (start 179.6375 114.8) (end 179.6375 112.2075) (width 0.5) (layer "F.Cu") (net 1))
 (segment (start 182.6275 107.07) (end 179.6375 110.06) (width 0.5) (layer "F.Cu") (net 1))
 (segment (start 176.125 101.36) (end 174.8775 101.36) (width 0.4) (layer "F.Cu") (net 1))
 (segment (start 178.3475 117.84) (end 178.3475 116.09) (width 0.5) (layer "F.Cu") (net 1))
 (segment (start 179.6375 110.06) (end 179.6375 112.88) (width 0.5) (layer "F.Cu") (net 1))
 (segment (start 179.6375 112.88) (end 179.6375 112.2075) (width 0.5) (layer "F.Cu") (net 1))
 (segment (start 179.6375 112.2075) (end 178.3075 112.2075) (width 0.5) (layer "F.Cu") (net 1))
 (via (at 182.825 101.3) (size 0.5) (drill 0.3) (layers "F.Cu" "B.Cu") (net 1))
 (via (at 176.125 101.36) (size 0.5) (drill 0.3) (layers "F.Cu" "B.Cu") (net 1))
 (segment (start 182.765 101.36) (end 182.825 101.3) (width 0.4) (layer "B.Cu") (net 1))
 (segment (start 176.125 101.36) (end 182.765 101.36) (width 0.4) (layer "B.Cu") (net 1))
 (segment (start 175.445 114.03) (end 178.305 114.03) (width 0.5) (layer "F.Cu") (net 2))
 (segment (start 178.305 114.03) (end 178.3075 114.0325) (width 0.5) (layer "F.Cu") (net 2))
 (segment (start 180.9575 106.27) (end 180.8475 106.38) (width 0.3) (layer "F.Cu") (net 7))
 (segment (start 180.6275 98.225) (end 180.8275 98.425) (width 0.3) (layer "F.Cu") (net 7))
 (segment (start 181.4375 99.41) (end 181.4375 105.79) (width 0.3) (layer "F.Cu") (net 7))
 (segment (start 181.2275 98.425) (end 181.4025 98.425) (width 0.3) (layer "F.Cu") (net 7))
 (segment (start 181.6275 97.33) (end 181.6275 98.2) (width 0.3) (layer "F.Cu") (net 7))
 (segment (start 181.4375 98.635) (end 181.4375 99.41) (width 0.3) (layer "F.Cu") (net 7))
 (segment (start 181.2275 98.425) (end 181.4375 98.635) (width 0.3) (layer "F.Cu") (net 7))
 (segment (start 181.4375 105.79) (end 180.9575 106.27) (width 0.3) (layer "F.Cu") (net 7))
 (segment (start 180.8275 98.425) (end 181.2275 98.425) (width 0.3) (layer "F.Cu") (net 7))
 (segment (start 181.6275 98.2) (end 181.4025 98.425) (width 0.3) (layer "F.Cu") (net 7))
 (segment (start 180.8475 106.38) (end 178.4975 106.38) (width 0.3) (layer "F.Cu") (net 7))
 (segment (start 180.6275 97.33) (end 180.6275 98.225) (width 0.3) (layer "F.Cu") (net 7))
 (segment (start 181.1275 96.235) (end 182.1275 96.235) (width 0.3) (layer "F.Cu") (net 8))
 (segment (start 181.1275 97.33) (end 181.1275 96.235) (width 0.3) (layer "F.Cu") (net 8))
 (segment (start 182.1275 96.235) (end 182.1275 97.33) (width 0.3) (layer "F.Cu") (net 8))
 (segment (start 181.9575 106.5) (end 180.9075 107.55) (width 0.3) (layer "F.Cu") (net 8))
 (segment (start 182.1275 98.44) (end 181.9575 98.61) (width 0.3) (layer "F.Cu") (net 8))
 (segment (start 180.9075 107.55) (end 180.8075 107.65) (width 0.3) (layer "F.Cu") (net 8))
 (segment (start 182.1275 97.33) (end 182.1275 98.44) (width 0.3) (layer "F.Cu") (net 8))
 (segment (start 180.8075 107.65) (end 178.4975 107.65) (width 0.3) (layer "F.Cu") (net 8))
 (segment (start 181.9575 98.61) (end 181.9575 106.5) (width 0.3) (layer "F.Cu") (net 8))
 (segment (start 182.6275 99.3) (end 182.7925 99.465) (width 0.3) (layer "F.Cu") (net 23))
 (segment (start 182.6275 97.33) (end 182.6275 99.3) (width 0.3) (layer "F.Cu") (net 23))
 (segment (start 179.6275 97.33) (end 179.6275 99.39) (width 0.3) (layer "F.Cu") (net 20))
 (segment (start 179.6275 99.39) (end 179.6925 99.455) (width 0.3) (layer "F.Cu") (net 20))
 (segment (start 183.4475 111.1975) (end 183.4475 112.2175) (width 0.5) (layer "F.Cu") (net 5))
 (segment (start 180.065 103.84) (end 178.4975 103.84) (width 0.5) (layer "F.Cu") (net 5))
 (segment (start 180.525 104.3) (end 180.065 103.84) (width 0.5) (layer "F.Cu") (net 5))
 (via (at 180.525 104.3) (size 0.5) (drill 0.3) (layers "F.Cu" "B.Cu") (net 5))
 (via (at 183.4475 111.1975) (size 0.8) (drill 0.4) (layers "F.Cu" "B.Cu") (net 5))
 (segment (start 180.525 108.275) (end 180.525 104.3) (width 0.5) (layer "B.Cu") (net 5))
 (segment (start 183.4475 111.1975) (end 180.525 108.275) (width 0.5) (layer "B.Cu") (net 5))
 (segment (start 179.5575 103.075) (end 179.5575 102.9075) (width 0.5) (layer "F.Cu") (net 4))
 (segment (start 180.85 112.17) (end 180.8975 112.2175) (width 0.5) (layer "F.Cu") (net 4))
 (segment (start 180.85 111.225) (end 180.85 112.17) (width 0.5) (layer "F.Cu") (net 4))
 (segment (start 179.5575 102.9075) (end 179.22 102.57) (width 0.5) (layer "F.Cu") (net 4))
 (segment (start 179.22 102.57) (end 178.4975 102.57) (width 0.5) (layer "F.Cu") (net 4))
 (via (at 180.85 111.225) (size 0.8) (drill 0.4) (layers "F.Cu" "B.Cu") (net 4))
 (via (at 179.5575 103.075) (size 0.5) (drill 0.3) (layers "F.Cu" "B.Cu") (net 4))
 (segment (start 179.5575 109.9325) (end 180.85 111.225) (width 0.5) (layer "B.Cu") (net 4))
 (segment (start 179.5575 103.075) (end 179.5575 109.9325) (width 0.5) (layer "B.Cu") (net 4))
 (segment (start 176.1875 108.98) (end 178.4375 108.98) (width 0.5) (layer "F.Cu") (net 9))
 (segment (start 178.4375 108.98) (end 178.4975 108.92) (width 0.5) (layer "F.Cu") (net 9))
 (segment (start 178.6775 108.98) (end 178.7375 108.92) (width 0.5) (layer "F.Cu") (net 9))
 (segment (start 186.82 114.04) (end 187.2475 113.6125) (width 0.5) (layer "F.Cu") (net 15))
 (segment (start 184.5875 105.11) (end 183.9975 105.11) (width 0.5) (layer "F.Cu") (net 15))
 (segment (start 187.2475 113.6125) (end 187.2475 104.74) (width 0.5) (layer "F.Cu") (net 15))
 (segment (start 187.2475 104.74) (end 186.9775 104.47) (width 0.5) (layer "F.Cu") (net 15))
 (segment (start 185.2275 104.47) (end 184.5875 105.11) (width 0.5) (layer "F.Cu") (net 15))
 (segment (start 186.9775 104.47) (end 185.2275 104.47) (width 0.5) (layer "F.Cu") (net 15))
 (segment (start 177.3075 111.38) (end 178.4975 110.19) (width 0.5) (layer "F.Cu") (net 10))
 (segment (start 176.1875 111.38) (end 177.3075 111.38) (width 0.5) (layer "F.Cu") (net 10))
 (segment (start 185.095 114.04) (end 185.9675 114.9125) (width 0.5) (layer "F.Cu") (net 19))
 (segment (start 185.9675 114.9125) (end 185.9675 117.84) (width 0.5) (layer "F.Cu") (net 19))
 (segment (start 183.4275 117.84) (end 183.4275 114.0825) (width 0.4) (layer "F.Cu") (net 21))
 (segment (start 180.8875 117.84) (end 180.8875 114.0625) (width 0.4) (layer "F.Cu") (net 18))
 (segment (start 185.7775 107.65) (end 186.0675 107.36) (width 0.5) (layer "F.Cu") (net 13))
 (segment (start 183.9975 107.65) (end 185.7775 107.65) (width 0.5) (layer "F.Cu") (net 13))
 (segment (start 183.9975 108.92) (end 185.8375 108.92) (width 0.5) (layer "F.Cu") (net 12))
 (segment (start 185.8375 108.92) (end 186.0675 109.15) (width 0.5) (layer "F.Cu") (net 12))
 (segment (start 185.3175 110.19) (end 186.0675 110.94) (width 0.5) (layer "F.Cu") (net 11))
 (segment (start 183.9975 110.19) (end 185.3175 110.19) (width 0.5) (layer "F.Cu") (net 11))
 (segment (start 185.76 105.84) (end 185.7975 105.84) (width 0.5) (layer "F.Cu") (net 14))
 (segment (start 185.7975 105.84) (end 186.0675 105.57) (width 0.5) (layer "F.Cu") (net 14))
 (segment (start 183.9975 106.38) (end 185.22 106.38) (width 0.5) (layer "F.Cu") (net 14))
 (segment (start 185.22 106.38) (end 185.76 105.84) (width 0.5) (layer "F.Cu") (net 14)))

